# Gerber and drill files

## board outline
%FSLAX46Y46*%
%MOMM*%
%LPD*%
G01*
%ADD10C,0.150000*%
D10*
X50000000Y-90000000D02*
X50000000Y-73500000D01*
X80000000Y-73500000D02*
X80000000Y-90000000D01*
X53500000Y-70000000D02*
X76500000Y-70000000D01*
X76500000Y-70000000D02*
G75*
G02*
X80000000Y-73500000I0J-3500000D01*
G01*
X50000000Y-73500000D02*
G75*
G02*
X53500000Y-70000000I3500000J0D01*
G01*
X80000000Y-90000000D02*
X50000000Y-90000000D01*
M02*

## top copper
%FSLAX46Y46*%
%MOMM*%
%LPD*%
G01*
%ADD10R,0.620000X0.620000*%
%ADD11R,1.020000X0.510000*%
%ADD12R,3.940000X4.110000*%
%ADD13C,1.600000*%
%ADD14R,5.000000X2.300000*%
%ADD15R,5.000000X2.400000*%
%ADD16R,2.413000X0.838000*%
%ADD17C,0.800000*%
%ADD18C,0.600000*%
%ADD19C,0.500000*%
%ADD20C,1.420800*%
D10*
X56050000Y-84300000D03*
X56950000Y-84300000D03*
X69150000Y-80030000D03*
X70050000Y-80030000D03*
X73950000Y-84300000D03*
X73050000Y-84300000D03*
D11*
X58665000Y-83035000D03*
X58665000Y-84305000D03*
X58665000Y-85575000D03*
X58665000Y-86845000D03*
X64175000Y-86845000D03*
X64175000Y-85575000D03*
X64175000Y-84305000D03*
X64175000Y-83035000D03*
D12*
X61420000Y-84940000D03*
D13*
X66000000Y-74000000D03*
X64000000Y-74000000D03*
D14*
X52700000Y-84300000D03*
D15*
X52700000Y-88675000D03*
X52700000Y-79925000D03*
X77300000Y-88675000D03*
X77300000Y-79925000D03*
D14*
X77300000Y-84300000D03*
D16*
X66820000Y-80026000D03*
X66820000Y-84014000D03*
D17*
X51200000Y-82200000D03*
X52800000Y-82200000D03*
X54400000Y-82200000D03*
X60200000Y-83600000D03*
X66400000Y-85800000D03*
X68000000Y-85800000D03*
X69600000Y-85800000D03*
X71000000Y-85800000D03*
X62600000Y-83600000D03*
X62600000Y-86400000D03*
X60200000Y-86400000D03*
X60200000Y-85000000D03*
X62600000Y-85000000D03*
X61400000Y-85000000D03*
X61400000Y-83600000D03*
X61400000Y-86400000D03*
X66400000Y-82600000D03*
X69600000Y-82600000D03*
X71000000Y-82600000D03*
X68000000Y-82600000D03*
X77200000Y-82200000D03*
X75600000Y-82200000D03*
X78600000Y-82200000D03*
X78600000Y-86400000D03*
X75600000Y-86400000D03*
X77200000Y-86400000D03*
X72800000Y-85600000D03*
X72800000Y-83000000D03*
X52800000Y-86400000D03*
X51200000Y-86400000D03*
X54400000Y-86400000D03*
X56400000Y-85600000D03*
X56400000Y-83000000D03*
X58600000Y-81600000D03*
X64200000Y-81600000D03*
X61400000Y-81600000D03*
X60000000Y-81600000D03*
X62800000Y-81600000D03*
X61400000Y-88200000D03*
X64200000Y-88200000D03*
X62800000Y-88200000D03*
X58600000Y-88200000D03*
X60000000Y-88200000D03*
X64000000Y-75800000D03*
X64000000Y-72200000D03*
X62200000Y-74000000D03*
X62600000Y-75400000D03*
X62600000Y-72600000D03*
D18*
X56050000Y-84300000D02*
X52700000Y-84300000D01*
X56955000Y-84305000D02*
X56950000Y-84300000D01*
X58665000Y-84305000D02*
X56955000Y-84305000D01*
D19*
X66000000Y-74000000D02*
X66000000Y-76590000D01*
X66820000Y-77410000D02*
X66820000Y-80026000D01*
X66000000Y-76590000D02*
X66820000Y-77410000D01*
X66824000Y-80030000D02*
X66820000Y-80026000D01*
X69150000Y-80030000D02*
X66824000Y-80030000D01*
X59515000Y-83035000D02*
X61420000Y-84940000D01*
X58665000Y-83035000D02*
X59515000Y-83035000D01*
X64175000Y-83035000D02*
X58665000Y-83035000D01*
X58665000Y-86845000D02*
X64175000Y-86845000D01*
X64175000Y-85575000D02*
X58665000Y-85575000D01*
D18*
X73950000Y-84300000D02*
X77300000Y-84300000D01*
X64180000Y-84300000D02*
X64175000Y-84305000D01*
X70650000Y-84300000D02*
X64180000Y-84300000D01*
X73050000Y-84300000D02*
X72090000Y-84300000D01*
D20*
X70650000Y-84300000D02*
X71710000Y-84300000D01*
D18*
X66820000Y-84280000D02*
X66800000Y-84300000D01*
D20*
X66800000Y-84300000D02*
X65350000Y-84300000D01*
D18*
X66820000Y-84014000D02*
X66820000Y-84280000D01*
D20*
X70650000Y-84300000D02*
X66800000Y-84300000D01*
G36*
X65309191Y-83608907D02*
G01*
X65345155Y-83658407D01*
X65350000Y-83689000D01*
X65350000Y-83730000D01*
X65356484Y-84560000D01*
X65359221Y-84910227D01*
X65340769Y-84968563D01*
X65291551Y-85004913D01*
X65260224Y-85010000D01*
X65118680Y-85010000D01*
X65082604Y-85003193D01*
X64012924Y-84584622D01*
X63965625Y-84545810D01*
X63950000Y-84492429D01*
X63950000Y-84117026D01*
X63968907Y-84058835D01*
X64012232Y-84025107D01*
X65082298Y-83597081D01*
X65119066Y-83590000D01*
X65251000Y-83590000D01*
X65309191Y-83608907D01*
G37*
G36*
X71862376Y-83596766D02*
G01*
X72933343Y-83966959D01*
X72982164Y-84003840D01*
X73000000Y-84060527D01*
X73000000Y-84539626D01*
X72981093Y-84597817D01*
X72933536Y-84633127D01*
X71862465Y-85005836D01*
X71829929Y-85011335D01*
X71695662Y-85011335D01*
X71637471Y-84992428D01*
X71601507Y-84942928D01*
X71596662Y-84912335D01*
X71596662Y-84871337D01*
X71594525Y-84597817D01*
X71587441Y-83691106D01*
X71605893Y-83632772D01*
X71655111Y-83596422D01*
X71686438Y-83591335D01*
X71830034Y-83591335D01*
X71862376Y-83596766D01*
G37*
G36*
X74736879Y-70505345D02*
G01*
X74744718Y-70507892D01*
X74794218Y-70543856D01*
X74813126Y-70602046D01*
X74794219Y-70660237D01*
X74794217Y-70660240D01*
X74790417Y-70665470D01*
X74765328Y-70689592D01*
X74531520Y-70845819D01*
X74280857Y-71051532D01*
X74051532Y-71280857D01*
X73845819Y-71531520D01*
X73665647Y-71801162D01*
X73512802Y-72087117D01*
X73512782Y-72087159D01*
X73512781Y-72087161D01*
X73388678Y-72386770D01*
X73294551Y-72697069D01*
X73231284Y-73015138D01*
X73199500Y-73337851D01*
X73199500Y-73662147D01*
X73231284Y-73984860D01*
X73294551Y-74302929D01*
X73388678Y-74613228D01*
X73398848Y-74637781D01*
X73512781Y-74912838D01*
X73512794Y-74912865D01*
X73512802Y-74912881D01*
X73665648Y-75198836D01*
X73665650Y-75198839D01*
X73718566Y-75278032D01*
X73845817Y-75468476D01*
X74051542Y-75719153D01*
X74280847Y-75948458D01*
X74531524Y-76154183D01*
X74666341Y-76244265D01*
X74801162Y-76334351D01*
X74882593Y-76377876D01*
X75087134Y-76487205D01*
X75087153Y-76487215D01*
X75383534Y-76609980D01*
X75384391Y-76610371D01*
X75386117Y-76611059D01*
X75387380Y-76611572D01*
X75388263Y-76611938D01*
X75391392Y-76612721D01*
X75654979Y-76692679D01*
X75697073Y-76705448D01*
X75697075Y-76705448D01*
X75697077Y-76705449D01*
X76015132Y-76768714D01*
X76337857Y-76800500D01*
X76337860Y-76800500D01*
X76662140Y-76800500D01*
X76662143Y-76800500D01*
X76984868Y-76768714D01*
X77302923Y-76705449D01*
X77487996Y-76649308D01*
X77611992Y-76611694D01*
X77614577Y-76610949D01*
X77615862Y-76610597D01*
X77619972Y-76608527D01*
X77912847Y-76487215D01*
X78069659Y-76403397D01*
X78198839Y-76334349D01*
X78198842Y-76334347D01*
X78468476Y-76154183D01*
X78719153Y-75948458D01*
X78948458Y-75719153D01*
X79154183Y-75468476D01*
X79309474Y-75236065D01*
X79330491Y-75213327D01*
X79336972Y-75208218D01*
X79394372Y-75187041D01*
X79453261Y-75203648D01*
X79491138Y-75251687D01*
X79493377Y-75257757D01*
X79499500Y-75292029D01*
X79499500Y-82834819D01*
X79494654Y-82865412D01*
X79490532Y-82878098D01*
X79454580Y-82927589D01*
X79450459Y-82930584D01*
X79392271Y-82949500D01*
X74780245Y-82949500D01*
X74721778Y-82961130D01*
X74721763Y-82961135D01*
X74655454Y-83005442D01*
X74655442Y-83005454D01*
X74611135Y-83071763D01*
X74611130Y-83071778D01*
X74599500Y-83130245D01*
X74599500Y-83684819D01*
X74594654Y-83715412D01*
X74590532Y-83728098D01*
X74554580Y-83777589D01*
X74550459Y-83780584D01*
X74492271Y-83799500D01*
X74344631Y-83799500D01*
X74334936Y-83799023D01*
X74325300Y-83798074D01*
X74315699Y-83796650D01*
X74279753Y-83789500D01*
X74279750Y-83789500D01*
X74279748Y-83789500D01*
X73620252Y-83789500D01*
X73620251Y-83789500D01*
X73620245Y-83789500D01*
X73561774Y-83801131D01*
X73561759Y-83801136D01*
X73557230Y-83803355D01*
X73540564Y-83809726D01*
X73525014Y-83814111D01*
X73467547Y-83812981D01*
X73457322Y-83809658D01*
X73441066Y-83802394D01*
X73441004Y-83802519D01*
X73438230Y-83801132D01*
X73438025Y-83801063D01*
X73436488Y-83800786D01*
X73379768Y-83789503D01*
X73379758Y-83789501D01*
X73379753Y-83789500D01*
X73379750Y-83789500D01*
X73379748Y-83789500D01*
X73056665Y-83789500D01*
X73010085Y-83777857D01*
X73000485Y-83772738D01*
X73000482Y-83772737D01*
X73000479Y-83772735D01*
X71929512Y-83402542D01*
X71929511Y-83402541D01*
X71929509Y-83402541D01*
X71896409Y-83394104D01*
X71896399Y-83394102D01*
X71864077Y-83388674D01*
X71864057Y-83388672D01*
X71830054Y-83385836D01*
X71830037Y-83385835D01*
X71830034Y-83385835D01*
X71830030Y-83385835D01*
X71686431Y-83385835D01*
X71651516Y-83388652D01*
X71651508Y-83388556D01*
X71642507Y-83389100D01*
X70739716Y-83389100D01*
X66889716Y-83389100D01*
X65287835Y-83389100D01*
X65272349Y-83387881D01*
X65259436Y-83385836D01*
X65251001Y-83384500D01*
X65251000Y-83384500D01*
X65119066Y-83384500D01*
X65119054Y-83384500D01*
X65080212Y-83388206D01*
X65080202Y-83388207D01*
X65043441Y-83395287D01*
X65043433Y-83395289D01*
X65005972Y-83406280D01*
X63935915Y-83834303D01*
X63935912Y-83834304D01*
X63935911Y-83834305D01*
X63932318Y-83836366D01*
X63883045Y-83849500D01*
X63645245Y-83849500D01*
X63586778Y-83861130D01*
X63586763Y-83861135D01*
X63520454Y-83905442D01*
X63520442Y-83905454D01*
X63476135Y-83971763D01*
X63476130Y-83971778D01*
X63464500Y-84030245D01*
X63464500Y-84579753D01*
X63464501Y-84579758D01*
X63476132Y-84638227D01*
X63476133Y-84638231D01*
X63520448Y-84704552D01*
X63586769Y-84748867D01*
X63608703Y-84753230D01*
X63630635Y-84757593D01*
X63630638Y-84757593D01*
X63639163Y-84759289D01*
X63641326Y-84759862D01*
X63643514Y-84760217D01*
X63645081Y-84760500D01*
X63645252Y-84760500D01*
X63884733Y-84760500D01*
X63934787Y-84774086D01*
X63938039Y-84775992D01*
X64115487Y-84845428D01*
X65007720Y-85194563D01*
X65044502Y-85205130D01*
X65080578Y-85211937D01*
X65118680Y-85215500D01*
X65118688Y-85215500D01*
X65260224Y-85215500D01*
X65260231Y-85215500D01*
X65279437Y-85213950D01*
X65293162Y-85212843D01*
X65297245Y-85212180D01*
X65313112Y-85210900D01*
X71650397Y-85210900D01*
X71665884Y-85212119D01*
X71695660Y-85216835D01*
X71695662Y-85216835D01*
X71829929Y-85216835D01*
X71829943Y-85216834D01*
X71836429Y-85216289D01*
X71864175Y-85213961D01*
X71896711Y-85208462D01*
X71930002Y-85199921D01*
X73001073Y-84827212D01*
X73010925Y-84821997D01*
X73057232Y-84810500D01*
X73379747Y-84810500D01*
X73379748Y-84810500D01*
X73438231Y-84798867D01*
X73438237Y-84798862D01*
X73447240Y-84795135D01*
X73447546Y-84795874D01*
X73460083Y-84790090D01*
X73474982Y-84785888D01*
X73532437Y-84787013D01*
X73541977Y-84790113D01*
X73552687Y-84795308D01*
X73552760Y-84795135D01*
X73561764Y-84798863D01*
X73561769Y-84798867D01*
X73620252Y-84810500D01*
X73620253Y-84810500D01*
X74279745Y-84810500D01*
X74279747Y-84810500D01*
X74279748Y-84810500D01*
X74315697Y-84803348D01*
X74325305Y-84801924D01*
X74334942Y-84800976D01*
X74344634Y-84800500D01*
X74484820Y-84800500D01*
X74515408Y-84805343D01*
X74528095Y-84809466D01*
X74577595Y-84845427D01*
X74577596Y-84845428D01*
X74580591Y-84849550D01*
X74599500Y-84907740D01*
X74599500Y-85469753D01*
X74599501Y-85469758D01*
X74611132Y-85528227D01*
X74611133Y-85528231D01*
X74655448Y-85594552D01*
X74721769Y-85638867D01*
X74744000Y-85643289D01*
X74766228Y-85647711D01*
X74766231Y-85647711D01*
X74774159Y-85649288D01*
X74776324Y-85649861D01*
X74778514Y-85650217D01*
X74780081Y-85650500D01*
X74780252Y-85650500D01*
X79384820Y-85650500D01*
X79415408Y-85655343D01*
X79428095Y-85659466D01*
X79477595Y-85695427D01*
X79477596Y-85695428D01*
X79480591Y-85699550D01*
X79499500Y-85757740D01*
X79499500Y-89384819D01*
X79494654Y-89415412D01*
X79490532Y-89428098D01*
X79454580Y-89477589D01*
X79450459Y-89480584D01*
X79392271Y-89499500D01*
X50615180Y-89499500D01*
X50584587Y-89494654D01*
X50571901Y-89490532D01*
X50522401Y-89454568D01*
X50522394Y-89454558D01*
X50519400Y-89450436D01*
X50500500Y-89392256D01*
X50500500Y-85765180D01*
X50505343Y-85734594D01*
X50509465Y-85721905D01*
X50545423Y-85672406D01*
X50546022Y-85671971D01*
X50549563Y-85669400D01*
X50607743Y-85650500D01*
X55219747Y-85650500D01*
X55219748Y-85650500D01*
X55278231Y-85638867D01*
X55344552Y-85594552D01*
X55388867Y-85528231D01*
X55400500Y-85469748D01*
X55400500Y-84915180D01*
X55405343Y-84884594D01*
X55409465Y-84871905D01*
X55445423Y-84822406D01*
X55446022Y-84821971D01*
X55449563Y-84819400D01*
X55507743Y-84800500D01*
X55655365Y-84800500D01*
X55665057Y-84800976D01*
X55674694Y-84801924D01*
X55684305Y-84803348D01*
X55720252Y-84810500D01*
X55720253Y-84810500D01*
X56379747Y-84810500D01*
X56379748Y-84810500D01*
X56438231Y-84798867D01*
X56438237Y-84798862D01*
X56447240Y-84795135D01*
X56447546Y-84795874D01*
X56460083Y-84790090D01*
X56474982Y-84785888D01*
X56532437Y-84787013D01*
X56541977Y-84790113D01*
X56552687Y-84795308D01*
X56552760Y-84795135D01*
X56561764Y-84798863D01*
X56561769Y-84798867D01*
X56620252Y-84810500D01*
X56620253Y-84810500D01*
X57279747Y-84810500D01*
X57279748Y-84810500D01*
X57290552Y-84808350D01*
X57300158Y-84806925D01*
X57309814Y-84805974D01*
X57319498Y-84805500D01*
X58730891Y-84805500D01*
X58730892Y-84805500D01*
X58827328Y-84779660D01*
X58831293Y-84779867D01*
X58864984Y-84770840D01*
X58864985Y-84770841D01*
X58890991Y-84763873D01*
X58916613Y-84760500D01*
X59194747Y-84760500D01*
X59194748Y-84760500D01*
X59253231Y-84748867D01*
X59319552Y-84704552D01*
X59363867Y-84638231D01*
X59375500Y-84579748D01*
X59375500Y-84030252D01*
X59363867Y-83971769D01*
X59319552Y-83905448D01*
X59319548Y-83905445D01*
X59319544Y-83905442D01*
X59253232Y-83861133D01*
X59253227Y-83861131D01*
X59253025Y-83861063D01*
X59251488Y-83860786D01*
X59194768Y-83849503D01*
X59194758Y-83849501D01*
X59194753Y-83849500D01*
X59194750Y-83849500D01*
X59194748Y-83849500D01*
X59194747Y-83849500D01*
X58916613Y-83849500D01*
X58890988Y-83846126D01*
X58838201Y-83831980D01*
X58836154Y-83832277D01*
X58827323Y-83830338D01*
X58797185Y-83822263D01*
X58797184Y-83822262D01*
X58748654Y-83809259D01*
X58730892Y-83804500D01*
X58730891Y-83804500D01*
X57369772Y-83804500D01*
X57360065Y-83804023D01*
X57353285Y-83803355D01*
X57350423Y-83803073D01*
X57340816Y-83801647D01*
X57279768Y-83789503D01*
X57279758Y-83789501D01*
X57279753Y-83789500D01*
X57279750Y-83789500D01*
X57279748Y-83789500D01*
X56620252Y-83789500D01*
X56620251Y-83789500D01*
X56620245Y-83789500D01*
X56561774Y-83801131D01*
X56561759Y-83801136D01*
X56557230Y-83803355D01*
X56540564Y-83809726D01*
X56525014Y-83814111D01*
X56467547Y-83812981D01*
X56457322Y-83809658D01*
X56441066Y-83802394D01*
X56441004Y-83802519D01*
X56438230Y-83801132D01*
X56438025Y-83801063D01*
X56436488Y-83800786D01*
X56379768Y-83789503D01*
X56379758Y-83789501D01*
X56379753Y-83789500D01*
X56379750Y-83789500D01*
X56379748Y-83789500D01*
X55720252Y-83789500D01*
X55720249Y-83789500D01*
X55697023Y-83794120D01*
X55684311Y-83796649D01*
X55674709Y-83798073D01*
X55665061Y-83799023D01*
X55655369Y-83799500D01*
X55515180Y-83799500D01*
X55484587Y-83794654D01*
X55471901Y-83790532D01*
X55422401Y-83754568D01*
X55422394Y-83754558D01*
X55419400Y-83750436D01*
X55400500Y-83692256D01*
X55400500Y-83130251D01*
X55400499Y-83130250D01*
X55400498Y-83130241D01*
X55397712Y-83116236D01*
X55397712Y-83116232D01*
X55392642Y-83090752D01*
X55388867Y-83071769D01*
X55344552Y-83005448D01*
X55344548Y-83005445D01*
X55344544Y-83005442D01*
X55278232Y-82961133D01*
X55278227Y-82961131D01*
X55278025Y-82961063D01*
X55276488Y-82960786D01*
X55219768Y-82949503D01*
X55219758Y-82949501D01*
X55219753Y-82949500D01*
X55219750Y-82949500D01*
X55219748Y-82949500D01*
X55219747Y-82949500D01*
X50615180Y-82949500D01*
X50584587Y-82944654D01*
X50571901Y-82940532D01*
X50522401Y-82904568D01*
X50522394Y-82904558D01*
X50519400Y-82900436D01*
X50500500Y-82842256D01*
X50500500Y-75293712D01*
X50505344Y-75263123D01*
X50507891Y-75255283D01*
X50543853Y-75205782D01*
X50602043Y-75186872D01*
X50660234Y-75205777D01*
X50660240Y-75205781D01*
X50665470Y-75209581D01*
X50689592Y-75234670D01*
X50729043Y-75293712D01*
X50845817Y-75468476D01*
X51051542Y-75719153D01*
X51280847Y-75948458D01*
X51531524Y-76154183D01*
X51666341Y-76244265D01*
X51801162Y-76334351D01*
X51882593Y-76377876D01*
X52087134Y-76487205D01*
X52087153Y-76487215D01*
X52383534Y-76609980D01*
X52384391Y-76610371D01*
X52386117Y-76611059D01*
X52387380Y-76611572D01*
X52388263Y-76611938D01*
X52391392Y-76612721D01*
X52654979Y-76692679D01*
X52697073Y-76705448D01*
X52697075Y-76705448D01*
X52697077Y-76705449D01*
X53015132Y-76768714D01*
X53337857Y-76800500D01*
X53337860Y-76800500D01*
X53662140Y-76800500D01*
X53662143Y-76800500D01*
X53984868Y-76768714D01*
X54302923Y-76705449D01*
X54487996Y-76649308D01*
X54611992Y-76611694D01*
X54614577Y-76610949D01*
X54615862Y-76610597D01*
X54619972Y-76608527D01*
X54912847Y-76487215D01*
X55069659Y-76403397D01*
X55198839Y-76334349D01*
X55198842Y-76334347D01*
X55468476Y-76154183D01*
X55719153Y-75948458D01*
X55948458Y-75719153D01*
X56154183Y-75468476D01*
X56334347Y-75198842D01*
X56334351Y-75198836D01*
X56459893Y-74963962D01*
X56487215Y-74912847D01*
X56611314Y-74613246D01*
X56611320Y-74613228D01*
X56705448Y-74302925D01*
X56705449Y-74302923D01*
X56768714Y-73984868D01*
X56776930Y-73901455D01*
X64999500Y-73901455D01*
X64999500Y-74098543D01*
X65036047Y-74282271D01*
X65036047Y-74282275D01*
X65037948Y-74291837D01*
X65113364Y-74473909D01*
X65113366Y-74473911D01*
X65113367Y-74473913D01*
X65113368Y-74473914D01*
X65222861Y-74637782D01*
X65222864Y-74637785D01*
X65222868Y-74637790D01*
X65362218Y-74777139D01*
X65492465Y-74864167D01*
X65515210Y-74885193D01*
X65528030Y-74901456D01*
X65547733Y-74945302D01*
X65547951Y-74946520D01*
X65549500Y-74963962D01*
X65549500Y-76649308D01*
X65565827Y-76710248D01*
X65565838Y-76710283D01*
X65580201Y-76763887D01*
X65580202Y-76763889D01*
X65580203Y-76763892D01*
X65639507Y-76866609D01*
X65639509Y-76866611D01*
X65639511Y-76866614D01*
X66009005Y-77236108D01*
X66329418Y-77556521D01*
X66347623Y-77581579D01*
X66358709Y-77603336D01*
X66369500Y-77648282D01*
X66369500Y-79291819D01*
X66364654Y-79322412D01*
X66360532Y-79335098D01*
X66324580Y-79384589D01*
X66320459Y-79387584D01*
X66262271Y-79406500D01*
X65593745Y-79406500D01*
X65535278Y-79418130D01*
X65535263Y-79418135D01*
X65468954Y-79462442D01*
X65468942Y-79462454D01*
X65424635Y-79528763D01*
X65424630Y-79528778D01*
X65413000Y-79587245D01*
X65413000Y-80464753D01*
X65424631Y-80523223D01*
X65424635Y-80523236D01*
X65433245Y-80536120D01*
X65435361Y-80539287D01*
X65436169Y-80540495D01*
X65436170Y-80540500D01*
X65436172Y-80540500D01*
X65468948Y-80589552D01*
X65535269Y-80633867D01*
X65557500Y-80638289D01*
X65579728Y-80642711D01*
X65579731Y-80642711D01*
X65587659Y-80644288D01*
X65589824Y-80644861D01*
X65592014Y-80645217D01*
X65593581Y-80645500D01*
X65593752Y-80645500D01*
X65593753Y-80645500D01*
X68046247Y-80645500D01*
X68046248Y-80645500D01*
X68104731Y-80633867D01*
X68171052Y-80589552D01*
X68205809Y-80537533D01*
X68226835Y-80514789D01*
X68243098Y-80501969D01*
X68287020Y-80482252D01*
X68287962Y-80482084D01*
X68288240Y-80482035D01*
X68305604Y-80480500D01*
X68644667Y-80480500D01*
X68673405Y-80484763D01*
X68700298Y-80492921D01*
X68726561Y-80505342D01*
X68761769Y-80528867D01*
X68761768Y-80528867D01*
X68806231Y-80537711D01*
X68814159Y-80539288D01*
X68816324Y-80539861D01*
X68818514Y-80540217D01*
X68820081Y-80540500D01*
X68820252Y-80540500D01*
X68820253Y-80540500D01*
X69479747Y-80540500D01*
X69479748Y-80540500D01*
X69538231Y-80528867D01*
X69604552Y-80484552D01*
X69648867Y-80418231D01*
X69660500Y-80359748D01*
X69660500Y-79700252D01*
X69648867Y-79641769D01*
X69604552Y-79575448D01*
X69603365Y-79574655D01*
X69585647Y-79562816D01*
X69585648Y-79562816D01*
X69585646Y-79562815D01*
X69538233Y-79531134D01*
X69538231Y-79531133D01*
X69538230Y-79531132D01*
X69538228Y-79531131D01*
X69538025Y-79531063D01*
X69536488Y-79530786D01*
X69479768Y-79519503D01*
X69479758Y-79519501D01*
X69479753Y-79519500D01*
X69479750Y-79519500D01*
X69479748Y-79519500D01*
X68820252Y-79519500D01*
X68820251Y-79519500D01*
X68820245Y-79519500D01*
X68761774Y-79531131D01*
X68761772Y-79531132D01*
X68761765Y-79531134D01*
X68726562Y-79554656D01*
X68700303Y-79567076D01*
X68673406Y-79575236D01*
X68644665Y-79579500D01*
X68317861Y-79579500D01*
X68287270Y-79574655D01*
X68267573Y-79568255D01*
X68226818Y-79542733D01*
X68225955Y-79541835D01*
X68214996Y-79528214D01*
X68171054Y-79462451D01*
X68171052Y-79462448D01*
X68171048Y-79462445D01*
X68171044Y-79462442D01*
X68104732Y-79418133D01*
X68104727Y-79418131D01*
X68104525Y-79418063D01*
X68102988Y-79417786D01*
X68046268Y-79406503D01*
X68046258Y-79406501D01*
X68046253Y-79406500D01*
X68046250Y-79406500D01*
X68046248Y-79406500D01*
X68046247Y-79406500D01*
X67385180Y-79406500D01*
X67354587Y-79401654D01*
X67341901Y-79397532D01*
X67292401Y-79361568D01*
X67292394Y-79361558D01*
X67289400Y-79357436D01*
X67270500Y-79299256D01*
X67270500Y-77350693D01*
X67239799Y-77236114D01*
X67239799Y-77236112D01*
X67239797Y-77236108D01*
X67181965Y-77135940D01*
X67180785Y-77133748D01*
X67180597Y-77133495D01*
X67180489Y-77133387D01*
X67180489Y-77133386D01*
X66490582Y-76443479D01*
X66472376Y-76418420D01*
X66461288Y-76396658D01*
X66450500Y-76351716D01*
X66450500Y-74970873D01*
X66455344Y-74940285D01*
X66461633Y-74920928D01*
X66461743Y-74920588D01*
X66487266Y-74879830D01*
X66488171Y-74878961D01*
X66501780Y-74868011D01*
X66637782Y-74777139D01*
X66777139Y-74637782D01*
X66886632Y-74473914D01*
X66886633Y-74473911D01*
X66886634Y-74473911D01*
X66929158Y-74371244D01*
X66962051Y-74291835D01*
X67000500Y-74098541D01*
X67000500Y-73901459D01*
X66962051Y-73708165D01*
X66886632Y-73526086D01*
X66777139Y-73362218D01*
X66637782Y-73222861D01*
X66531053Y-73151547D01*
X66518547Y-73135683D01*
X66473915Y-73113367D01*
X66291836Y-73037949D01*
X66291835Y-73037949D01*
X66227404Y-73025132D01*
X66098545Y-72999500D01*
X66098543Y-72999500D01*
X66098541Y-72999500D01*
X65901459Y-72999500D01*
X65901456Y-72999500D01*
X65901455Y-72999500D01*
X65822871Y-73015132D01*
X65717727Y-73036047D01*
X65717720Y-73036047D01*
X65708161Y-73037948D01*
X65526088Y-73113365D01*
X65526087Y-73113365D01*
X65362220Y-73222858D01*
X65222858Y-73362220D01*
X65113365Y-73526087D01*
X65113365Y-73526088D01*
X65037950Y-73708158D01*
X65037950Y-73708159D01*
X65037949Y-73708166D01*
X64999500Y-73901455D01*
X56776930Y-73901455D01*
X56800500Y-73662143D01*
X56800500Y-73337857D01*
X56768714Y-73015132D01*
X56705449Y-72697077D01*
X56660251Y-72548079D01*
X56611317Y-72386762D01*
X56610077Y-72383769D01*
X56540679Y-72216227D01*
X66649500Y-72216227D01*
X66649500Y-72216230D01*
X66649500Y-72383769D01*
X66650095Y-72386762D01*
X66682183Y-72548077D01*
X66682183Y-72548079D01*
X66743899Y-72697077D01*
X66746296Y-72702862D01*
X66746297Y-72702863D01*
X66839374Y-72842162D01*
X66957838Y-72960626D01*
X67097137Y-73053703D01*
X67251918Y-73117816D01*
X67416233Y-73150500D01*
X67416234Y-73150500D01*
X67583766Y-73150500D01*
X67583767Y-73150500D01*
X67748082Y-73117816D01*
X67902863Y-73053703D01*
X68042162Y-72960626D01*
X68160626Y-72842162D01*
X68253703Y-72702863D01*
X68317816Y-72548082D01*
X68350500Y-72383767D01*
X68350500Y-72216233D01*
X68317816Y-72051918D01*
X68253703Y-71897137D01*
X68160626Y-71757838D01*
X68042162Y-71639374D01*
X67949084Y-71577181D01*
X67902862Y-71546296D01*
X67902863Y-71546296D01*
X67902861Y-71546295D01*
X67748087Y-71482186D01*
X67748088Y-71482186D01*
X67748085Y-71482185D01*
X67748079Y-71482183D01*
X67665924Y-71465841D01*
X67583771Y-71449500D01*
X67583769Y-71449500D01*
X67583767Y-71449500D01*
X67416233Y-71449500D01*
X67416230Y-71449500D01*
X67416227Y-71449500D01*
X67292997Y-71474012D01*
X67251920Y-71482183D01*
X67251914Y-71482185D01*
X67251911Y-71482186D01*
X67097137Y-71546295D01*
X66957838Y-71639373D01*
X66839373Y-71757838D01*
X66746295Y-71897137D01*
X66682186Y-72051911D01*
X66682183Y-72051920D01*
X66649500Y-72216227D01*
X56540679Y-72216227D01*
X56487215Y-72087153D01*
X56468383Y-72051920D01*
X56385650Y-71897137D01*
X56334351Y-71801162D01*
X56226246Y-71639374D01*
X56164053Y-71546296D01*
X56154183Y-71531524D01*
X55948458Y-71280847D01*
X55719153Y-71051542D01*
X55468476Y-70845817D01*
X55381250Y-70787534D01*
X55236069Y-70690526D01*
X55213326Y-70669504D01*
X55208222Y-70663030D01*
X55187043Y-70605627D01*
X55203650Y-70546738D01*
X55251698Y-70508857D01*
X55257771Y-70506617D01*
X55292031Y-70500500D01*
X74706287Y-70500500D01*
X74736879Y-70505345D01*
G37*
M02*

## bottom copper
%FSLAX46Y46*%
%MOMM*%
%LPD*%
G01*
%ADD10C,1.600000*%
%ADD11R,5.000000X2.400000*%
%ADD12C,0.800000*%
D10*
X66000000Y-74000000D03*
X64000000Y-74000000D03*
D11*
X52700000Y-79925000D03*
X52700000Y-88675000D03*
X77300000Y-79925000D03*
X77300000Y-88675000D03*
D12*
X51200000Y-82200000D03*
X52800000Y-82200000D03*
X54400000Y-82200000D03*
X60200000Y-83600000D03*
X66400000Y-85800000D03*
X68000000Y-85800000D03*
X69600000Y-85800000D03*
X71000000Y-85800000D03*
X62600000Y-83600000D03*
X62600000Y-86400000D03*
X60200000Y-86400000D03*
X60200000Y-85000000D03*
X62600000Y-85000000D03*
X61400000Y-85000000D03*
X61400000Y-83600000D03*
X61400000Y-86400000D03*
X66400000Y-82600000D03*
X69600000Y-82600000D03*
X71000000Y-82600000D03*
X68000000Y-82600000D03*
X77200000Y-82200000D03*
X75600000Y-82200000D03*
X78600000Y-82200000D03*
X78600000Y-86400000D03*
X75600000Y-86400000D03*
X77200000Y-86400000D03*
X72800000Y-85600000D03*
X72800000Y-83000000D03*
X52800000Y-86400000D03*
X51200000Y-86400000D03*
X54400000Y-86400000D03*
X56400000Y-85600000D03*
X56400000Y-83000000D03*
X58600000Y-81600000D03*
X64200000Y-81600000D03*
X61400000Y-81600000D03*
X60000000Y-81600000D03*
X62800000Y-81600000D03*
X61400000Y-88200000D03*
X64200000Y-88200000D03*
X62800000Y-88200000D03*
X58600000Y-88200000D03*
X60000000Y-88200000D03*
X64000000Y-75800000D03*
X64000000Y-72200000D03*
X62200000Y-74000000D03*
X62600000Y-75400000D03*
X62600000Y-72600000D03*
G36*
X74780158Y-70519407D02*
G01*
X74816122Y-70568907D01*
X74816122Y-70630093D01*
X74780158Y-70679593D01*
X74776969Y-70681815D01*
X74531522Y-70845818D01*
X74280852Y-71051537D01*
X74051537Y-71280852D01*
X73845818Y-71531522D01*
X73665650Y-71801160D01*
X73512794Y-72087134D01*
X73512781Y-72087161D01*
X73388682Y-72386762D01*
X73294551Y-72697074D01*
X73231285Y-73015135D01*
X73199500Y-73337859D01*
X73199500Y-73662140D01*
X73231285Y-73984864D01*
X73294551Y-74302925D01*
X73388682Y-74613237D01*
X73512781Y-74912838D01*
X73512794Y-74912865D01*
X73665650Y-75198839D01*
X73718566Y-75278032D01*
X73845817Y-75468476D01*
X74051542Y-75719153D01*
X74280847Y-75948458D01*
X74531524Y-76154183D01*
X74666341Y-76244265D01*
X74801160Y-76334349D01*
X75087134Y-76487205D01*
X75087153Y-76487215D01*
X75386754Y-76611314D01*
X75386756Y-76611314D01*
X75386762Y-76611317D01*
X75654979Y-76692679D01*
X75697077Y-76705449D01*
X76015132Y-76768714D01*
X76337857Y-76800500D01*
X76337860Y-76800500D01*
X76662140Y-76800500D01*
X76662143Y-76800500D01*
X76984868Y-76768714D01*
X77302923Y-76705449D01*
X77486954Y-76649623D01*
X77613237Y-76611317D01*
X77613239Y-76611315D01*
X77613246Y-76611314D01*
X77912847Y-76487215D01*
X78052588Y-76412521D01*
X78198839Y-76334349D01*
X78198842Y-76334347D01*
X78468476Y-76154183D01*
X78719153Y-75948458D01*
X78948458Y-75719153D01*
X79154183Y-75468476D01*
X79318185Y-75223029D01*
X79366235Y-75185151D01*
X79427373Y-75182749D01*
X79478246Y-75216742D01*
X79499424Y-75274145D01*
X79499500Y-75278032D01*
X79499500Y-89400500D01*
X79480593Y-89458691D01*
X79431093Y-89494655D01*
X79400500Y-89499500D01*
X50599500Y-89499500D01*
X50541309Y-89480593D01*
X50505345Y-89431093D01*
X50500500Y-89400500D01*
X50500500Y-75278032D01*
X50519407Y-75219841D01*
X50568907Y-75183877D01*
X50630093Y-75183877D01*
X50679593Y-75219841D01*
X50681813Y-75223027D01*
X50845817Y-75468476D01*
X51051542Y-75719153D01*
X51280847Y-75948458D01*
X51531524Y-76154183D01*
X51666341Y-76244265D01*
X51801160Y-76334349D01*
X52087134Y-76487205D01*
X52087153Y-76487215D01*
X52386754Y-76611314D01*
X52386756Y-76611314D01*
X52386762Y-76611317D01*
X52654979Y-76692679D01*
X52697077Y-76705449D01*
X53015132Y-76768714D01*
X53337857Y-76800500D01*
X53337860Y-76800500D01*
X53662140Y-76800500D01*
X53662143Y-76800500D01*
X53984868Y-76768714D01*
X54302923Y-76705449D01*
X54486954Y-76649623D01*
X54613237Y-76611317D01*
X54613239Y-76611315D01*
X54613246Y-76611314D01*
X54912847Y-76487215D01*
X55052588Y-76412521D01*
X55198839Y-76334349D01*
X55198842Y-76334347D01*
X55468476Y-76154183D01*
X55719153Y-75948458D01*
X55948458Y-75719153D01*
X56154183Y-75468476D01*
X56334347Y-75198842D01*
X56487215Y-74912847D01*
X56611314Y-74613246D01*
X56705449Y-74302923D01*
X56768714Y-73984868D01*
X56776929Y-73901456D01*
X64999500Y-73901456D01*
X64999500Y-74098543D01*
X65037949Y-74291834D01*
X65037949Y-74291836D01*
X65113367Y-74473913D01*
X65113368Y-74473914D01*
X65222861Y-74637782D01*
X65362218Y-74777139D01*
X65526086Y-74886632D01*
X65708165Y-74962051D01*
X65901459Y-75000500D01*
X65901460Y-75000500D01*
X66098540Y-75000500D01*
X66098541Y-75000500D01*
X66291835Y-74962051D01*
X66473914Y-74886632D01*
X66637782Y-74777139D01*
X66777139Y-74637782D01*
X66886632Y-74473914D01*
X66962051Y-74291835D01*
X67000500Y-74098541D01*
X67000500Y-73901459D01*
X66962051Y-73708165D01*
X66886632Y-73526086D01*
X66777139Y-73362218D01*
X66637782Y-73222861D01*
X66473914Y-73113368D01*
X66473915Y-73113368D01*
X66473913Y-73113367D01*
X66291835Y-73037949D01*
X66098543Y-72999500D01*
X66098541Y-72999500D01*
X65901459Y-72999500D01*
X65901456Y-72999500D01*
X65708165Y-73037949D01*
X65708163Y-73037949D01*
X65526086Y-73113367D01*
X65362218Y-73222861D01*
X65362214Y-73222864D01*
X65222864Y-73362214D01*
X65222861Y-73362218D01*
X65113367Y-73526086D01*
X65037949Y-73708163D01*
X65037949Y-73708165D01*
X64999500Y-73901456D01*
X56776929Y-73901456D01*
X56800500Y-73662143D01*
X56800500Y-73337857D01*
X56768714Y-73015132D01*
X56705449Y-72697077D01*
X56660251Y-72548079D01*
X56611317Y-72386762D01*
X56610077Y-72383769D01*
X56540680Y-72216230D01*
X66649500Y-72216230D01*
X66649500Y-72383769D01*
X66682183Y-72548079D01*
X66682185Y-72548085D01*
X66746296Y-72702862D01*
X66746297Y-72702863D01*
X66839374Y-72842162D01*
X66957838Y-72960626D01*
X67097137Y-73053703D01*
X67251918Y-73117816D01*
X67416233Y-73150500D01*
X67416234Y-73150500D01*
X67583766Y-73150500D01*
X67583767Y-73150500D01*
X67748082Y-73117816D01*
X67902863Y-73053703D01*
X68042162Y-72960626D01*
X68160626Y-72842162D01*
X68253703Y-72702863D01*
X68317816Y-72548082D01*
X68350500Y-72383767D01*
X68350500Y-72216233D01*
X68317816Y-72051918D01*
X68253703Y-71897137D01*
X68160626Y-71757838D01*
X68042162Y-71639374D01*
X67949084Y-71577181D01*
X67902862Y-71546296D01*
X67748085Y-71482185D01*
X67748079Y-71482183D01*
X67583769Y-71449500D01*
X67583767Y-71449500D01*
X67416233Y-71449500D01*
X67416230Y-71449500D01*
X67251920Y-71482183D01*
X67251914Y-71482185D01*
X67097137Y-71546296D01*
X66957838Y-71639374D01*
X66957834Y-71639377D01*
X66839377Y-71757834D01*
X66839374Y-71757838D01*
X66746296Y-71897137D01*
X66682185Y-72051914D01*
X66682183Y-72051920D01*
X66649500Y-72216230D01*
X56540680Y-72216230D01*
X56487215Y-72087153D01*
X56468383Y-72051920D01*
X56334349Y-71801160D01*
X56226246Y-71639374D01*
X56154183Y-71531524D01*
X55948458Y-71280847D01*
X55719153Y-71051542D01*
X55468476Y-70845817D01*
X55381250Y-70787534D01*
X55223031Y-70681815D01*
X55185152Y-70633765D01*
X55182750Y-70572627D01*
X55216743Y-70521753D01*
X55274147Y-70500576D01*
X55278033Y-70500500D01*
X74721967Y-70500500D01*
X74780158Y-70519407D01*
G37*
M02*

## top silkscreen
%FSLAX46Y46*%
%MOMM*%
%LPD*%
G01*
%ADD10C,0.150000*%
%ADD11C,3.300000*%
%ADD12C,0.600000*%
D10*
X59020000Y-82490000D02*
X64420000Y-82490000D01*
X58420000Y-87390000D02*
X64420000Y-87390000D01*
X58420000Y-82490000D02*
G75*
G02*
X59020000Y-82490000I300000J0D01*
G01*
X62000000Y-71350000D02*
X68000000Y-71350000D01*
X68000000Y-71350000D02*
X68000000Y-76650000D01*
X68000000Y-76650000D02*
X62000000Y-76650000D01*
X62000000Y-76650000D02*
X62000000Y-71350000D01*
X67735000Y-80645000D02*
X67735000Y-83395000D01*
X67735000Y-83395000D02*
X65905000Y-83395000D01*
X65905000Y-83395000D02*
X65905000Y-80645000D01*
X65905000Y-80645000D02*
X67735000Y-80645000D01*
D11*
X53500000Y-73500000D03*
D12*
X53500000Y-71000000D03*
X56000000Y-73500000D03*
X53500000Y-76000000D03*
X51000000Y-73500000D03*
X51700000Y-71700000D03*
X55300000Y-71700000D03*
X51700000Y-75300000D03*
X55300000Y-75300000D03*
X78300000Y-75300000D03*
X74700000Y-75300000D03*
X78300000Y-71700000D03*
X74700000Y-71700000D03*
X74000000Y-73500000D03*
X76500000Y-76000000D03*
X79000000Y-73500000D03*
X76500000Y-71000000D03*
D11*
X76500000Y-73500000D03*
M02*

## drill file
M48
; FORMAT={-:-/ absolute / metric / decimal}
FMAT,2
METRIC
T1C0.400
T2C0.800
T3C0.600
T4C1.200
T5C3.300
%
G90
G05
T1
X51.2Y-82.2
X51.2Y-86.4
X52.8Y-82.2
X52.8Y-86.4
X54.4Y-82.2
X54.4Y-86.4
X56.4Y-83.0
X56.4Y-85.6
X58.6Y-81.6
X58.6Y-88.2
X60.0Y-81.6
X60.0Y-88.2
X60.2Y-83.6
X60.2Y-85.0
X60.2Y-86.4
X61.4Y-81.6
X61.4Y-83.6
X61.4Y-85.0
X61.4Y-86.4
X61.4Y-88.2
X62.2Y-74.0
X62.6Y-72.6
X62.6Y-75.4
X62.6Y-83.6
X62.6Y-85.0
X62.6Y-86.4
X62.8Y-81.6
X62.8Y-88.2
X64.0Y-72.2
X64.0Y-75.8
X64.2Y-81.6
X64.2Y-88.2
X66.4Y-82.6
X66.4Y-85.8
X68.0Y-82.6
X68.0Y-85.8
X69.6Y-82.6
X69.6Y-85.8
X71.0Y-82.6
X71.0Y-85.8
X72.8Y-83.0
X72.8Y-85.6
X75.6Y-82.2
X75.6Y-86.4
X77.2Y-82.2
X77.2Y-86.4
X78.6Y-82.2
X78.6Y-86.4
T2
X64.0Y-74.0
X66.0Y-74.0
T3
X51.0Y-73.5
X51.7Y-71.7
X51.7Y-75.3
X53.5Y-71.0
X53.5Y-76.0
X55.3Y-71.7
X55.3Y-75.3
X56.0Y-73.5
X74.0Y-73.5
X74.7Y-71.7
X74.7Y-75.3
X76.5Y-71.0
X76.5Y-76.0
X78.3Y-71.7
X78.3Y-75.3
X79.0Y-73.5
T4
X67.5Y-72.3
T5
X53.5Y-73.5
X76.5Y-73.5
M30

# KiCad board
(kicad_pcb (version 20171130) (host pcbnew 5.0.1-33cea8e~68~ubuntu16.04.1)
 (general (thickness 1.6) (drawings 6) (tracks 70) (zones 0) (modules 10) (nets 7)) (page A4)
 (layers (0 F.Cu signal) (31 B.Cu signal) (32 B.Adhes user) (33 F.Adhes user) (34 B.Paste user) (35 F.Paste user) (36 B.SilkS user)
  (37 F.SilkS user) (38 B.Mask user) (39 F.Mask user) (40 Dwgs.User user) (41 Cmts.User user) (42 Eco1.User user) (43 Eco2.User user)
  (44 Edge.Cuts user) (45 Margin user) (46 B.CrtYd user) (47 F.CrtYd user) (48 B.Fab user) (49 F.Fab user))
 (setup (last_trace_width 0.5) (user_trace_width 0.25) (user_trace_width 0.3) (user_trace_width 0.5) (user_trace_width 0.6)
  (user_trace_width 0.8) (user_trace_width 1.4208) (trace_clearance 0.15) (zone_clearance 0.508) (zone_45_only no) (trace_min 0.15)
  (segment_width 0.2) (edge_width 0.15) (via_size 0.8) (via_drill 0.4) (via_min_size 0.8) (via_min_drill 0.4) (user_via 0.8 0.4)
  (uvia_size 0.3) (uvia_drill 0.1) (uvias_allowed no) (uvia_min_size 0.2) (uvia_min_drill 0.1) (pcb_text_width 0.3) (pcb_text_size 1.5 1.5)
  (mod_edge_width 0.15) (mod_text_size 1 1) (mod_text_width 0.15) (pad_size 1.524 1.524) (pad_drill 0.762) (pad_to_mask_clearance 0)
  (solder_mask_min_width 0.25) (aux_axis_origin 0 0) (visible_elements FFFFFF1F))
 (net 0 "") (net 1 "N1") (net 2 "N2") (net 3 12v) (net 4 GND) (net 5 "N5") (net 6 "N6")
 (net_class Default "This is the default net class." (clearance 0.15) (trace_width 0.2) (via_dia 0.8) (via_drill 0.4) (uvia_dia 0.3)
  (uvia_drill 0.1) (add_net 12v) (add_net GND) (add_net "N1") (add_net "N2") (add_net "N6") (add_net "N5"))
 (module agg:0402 (layer F.Cu) (at 56.5 84.3)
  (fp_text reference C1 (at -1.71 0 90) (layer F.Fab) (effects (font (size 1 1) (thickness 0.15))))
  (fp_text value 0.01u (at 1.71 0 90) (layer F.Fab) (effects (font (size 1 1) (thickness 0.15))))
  (pad 1 smd rect (at -0.45 0) (size 0.62 0.62) (layers F.Cu F.Paste F.Mask) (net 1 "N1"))
  (pad 2 smd rect (at 0.45 0) (size 0.62 0.62) (layers F.Cu F.Paste F.Mask) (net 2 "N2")))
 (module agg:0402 (layer F.Cu) (at 69.6 80.03)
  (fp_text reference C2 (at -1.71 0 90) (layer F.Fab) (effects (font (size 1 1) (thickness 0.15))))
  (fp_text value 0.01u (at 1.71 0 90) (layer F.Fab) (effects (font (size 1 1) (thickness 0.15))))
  (pad 1 smd rect (at -0.45 0) (size 0.62 0.62) (layers F.Cu F.Paste F.Mask) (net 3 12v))
  (pad 2 smd rect (at 0.45 0) (size 0.62 0.62) (layers F.Cu F.Paste F.Mask) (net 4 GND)))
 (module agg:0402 (layer F.Cu) (at 73.5 84.3)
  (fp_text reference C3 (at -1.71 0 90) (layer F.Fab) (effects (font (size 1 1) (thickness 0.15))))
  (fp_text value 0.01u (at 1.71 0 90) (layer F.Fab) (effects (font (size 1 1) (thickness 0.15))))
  (pad 2 smd rect (at 0.45 0) (size 0.62 0.62) (layers F.Cu F.Paste F.Mask) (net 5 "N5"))
  (pad 1 smd rect (at -0.45 0) (size 0.62 0.62) (layers F.Cu F.Paste F.Mask) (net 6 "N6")))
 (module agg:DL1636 (layer F.Cu) (at 61.42 84.94)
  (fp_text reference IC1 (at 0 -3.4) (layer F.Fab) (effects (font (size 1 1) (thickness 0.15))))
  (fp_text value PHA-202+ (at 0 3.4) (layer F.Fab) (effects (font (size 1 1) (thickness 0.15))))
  (fp_line (start -2.4 -2.45) (end 3 -2.45) (layer F.SilkS) (width 0.15))
  (fp_line (start -3 2.45) (end 3 2.45) (layer F.SilkS) (width 0.15))
  (fp_arc (start -2.7 -2.45) (end -3 -2.45) (angle 180) (layer F.SilkS) (width 0.15))
  (pad 1 smd rect (at -2.755 -1.905) (size 1.02 0.51) (layers F.Cu F.Paste F.Mask) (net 4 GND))
  (pad 2 smd rect (at -2.755 -0.635) (size 1.02 0.51) (layers F.Cu F.Paste F.Mask) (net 2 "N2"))
  (pad 3 smd rect (at -2.755 0.635) (size 1.02 0.51) (layers F.Cu F.Paste F.Mask) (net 4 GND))
  (pad 4 smd rect (at -2.755 1.905) (size 1.02 0.51) (layers F.Cu F.Paste F.Mask) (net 4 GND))
  (pad 5 smd rect (at 2.755 1.905) (size 1.02 0.51) (layers F.Cu F.Paste F.Mask) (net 4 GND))
  (pad 6 smd rect (at 2.755 0.635) (size 1.02 0.51) (layers F.Cu F.Paste F.Mask) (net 4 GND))
  (pad 7 smd rect (at 2.755 -0.635) (size 1.02 0.51) (layers F.Cu F.Paste F.Mask) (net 6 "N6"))
  (pad 8 smd rect (at 2.755 -1.905) (size 1.02 0.51) (layers F.Cu F.Paste F.Mask) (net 4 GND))
  (pad EP smd rect (at 0 0) (size 3.94 4.11) (layers F.Cu F.Paste F.Mask) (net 4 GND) (solder_mask_margin 0.001) (solder_paste_margin 0.001)))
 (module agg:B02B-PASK (layer F.Cu) (at 65 74)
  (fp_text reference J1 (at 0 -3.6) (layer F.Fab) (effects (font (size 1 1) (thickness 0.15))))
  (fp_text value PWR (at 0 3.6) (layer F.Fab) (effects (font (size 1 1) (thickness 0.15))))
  (fp_line (start -3 -2.65) (end 3 -2.65) (layer F.SilkS) (width 0.15))
  (fp_line (start 3 -2.65) (end 3 2.65) (layer F.SilkS) (width 0.15))
  (fp_line (start 3 2.65) (end -3 2.65) (layer F.SilkS) (width 0.15))
  (fp_line (start -3 2.65) (end -3 -2.65) (layer F.SilkS) (width 0.15))
  (pad "" np_thru_hole circle (at 2.5 -1.7) (size 1.2 1.2) (drill 1.2) (layers *.Mask))
  (pad 1 thru_hole circle (at 1 0) (size 1.6 1.6) (drill 0.8) (layers *.Cu *.Mask) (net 3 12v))
  (pad 2 thru_hole circle (at -1 0) (size 1.6 1.6) (drill 0.8) (layers *.Cu *.Mask) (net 4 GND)))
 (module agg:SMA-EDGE (layer F.Cu) (at 52.7 84.3 90)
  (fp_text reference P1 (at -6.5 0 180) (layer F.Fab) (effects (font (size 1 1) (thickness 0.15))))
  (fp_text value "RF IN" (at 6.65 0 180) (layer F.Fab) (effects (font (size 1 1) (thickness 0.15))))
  (pad 1 smd rect (at 0 0 90) (size 2.3 5) (layers F.Cu F.Paste F.Mask) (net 1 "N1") (zone_connect 2))
  (pad 2 smd rect (at 4.375 0 90) (size 2.4 5) (layers B.Cu B.Paste B.Mask) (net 4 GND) (zone_connect 2))
  (pad 2 smd rect (at -4.375 0 90) (size 2.4 5) (layers B.Cu B.Paste B.Mask) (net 4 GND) (zone_connect 2))
  (pad 2 smd rect (at -4.375 0 90) (size 2.4 5) (layers F.Cu F.Paste F.Mask) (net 4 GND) (zone_connect 2))
  (pad 2 smd rect (at 4.375 0 90) (size 2.4 5) (layers F.Cu F.Paste F.Mask) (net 4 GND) (zone_connect 2)))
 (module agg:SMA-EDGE (layer F.Cu) (at 77.3 84.3 270)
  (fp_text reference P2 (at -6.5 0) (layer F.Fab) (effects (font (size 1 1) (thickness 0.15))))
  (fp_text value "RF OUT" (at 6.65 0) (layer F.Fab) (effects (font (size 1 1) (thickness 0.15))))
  (pad 2 smd rect (at 4.375 0 270) (size 2.4 5) (layers F.Cu F.Paste F.Mask) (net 4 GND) (zone_connect 2))
  (pad 2 smd rect (at -4.375 0 270) (size 2.4 5) (layers F.Cu F.Paste F.Mask) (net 4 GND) (zone_connect 2))
  (pad 2 smd rect (at -4.375 0 270) (size 2.4 5) (layers B.Cu B.Paste B.Mask) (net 4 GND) (zone_connect 2))
  (pad 2 smd rect (at 4.375 0 270) (size 2.4 5) (layers B.Cu B.Paste B.Mask) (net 4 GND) (zone_connect 2))
  (pad 1 smd rect (at 0 0 270) (size 2.3 5) (layers F.Cu F.Paste F.Mask) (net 5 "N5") (zone_connect 2)))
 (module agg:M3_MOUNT (layer F.Cu) (at 53.5 73.5)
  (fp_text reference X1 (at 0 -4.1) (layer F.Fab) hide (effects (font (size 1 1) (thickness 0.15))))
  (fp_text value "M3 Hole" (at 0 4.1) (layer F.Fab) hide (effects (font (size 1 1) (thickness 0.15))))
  (pad "" np_thru_hole circle (at 0 0) (size 3.3 3.3) (drill 3.3) (layers *.Cu *.Mask F.SilkS) (solder_mask_margin 1.5) (clearance 1.65))
  (pad "" np_thru_hole circle (at 0 -2.5) (size 0.6 0.6) (drill 0.6) (layers *.Cu *.Mask F.SilkS))
  (pad "" np_thru_hole circle (at 2.5 0) (size 0.6 0.6) (drill 0.6) (layers *.Cu *.Mask F.SilkS))
  (pad "" np_thru_hole circle (at 0 2.5) (size 0.6 0.6) (drill 0.6) (layers *.Cu *.Mask F.SilkS))
  (pad "" np_thru_hole circle (at -2.5 0) (size 0.6 0.6) (drill 0.6) (layers *.Cu *.Mask F.SilkS))
  (pad "" np_thru_hole circle (at -1.8 -1.8) (size 0.6 0.6) (drill 0.6) (layers *.Cu *.Mask F.SilkS))
  (pad "" np_thru_hole circle (at 1.8 -1.8) (size 0.6 0.6) (drill 0.6) (layers *.Cu *.Mask F.SilkS))
  (pad "" np_thru_hole circle (at -1.8 1.8) (size 0.6 0.6) (drill 0.6) (layers *.Cu *.Mask F.SilkS))
  (pad "" np_thru_hole circle (at 1.8 1.8) (size 0.6 0.6) (drill 0.6) (layers *.Cu *.Mask F.SilkS)))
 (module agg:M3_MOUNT (layer F.Cu) (at 76.5 73.5)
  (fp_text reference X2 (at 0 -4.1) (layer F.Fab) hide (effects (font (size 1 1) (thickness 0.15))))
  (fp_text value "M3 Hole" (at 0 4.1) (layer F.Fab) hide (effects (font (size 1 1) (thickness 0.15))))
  (pad "" np_thru_hole circle (at 1.8 1.8) (size 0.6 0.6) (drill 0.6) (layers *.Cu *.Mask F.SilkS))
  (pad "" np_thru_hole circle (at -1.8 1.8) (size 0.6 0.6) (drill 0.6) (layers *.Cu *.Mask F.SilkS))
  (pad "" np_thru_hole circle (at 1.8 -1.8) (size 0.6 0.6) (drill 0.6) (layers *.Cu *.Mask F.SilkS))
  (pad "" np_thru_hole circle (at -1.8 -1.8) (size 0.6 0.6) (drill 0.6) (layers *.Cu *.Mask F.SilkS))
  (pad "" np_thru_hole circle (at -2.5 0) (size 0.6 0.6) (drill 0.6) (layers *.Cu *.Mask F.SilkS))
  (pad "" np_thru_hole circle (at 0 2.5) (size 0.6 0.6) (drill 0.6) (layers *.Cu *.Mask F.SilkS))
  (pad "" np_thru_hole circle (at 2.5 0) (size 0.6 0.6) (drill 0.6) (layers *.Cu *.Mask F.SilkS))
  (pad "" np_thru_hole circle (at 0 -2.5) (size 0.6 0.6) (drill 0.6) (layers *.Cu *.Mask F.SilkS))
  (pad "" np_thru_hole circle (at 0 0) (size 3.3 3.3) (drill 3.3) (layers *.Cu *.Mask F.SilkS) (solder_mask_margin 1.5) (clearance 1.65)))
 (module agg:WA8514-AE (layer F.Cu) (at 66.82 82.02 270)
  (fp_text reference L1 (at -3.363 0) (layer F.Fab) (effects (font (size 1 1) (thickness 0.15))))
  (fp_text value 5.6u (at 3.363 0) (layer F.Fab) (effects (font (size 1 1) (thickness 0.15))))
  (fp_line (start -1.375 -0.915) (end 1.375 -0.915) (layer F.SilkS) (width 0.15))
  (fp_line (start 1.375 -0.915) (end 1.375 0.915) (layer F.SilkS) (width 0.15))
  (fp_line (start 1.375 0.915) (end -1.375 0.915) (layer F.SilkS) (width 0.15))
  (fp_line (start -1.375 0.915) (end -1.375 -0.915) (layer F.SilkS) (width 0.15))
  (pad 1 smd rect (at -1.994 0 270) (size 0.838 2.413) (layers F.Cu F.Paste F.Mask) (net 3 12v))
  (pad 2 smd rect (at 1.994 0 270) (size 0.838 2.413) (layers F.Cu F.Paste F.Mask) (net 6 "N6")))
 (gr_line (start 50 90) (end 50 73.5) (layer Edge.Cuts) (width 0.15))
 (gr_line (start 80 73.5) (end 80 90) (layer Edge.Cuts) (width 0.15))
 (gr_line (start 53.5 70) (end 76.5 70) (layer Edge.Cuts) (width 0.15))
 (gr_arc (start 76.5 73.5) (end 80 73.5) (angle -90) (layer Edge.Cuts) (width 0.15))
 (gr_arc (start 53.5 73.5) (end 53.5 70) (angle -90) (layer Edge.Cuts) (width 0.15))
 (gr_line (start 80 90) (end 50 90) (layer Edge.Cuts) (width 0.15))
 (segment (start 56.05 84.3) (end 52.7 84.3) (width 0.6) (layer F.Cu) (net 1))
 (segment (start 56.955 84.305) (end 56.95 84.3) (width 0.6) (layer F.Cu) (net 2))
 (segment (start 58.665 84.305) (end 56.955 84.305) (width 0.6) (layer F.Cu) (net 2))
 (segment (start 66 74) (end 66 76.59) (width 0.5) (layer F.Cu) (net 3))
 (segment (start 66.82 77.41) (end 66.82 80.026) (width 0.5) (layer F.Cu) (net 3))
 (segment (start 66 76.59) (end 66.82 77.41) (width 0.5) (layer F.Cu) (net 3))
 (segment (start 66.824 80.03) (end 66.82 80.026) (width 0.5) (layer F.Cu) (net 3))
 (segment (start 69.15 80.03) (end 66.824 80.03) (width 0.5) (layer F.Cu) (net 3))
 (segment (start 59.515 83.035) (end 61.42 84.94) (width 0.5) (layer F.Cu) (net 4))
 (segment (start 58.665 83.035) (end 59.515 83.035) (width 0.5) (layer F.Cu) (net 4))
 (segment (start 64.175 83.035) (end 58.665 83.035) (width 0.5) (layer F.Cu) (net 4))
 (segment (start 58.665 86.845) (end 64.175 86.845) (width 0.5) (layer F.Cu) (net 4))
 (segment (start 64.175 85.575) (end 58.665 85.575) (width 0.5) (layer F.Cu) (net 4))
 (via (at 51.2 82.2) (size 0.8) (drill 0.4) (layers F.Cu B.Cu) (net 4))
 (via (at 52.8 82.2) (size 0.8) (drill 0.4) (layers F.Cu B.Cu) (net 4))
 (via (at 54.4 82.2) (size 0.8) (drill 0.4) (layers F.Cu B.Cu) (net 4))
 (via (at 60.2 83.6) (size 0.8) (drill 0.4) (layers F.Cu B.Cu) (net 4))
 (via (at 66.4 85.8) (size 0.8) (drill 0.4) (layers F.Cu B.Cu) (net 4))
 (via (at 68 85.8) (size 0.8) (drill 0.4) (layers F.Cu B.Cu) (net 4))
 (via (at 69.6 85.8) (size 0.8) (drill 0.4) (layers F.Cu B.Cu) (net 4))
 (via (at 71 85.8) (size 0.8) (drill 0.4) (layers F.Cu B.Cu) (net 4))
 (via (at 62.6 83.6) (size 0.8) (drill 0.4) (layers F.Cu B.Cu) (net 4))
 (via (at 62.6 86.4) (size 0.8) (drill 0.4) (layers F.Cu B.Cu) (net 4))
 (via (at 60.2 86.4) (size 0.8) (drill 0.4) (layers F.Cu B.Cu) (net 4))
 (via (at 60.2 85) (size 0.8) (drill 0.4) (layers F.Cu B.Cu) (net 4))
 (via (at 62.6 85) (size 0.8) (drill 0.4) (layers F.Cu B.Cu) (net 4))
 (via (at 61.4 85) (size 0.8) (drill 0.4) (layers F.Cu B.Cu) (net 4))
 (via (at 61.4 83.6) (size 0.8) (drill 0.4) (layers F.Cu B.Cu) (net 4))
 (via (at 61.4 86.4) (size 0.8) (drill 0.4) (layers F.Cu B.Cu) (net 4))
 (via (at 66.4 82.6) (size 0.8) (drill 0.4) (layers F.Cu B.Cu) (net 4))
 (via (at 69.6 82.6) (size 0.8) (drill 0.4) (layers F.Cu B.Cu) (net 4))
 (via (at 71 82.6) (size 0.8) (drill 0.4) (layers F.Cu B.Cu) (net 4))
 (via (at 68 82.6) (size 0.8) (drill 0.4) (layers F.Cu B.Cu) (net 4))
 (via (at 77.2 82.2) (size 0.8) (drill 0.4) (layers F.Cu B.Cu) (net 4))
 (via (at 75.6 82.2) (size 0.8) (drill 0.4) (layers F.Cu B.Cu) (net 4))
 (via (at 78.6 82.2) (size 0.8) (drill 0.4) (layers F.Cu B.Cu) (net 4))
 (via (at 78.6 86.4) (size 0.8) (drill 0.4) (layers F.Cu B.Cu) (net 4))
 (via (at 75.6 86.4) (size 0.8) (drill 0.4) (layers F.Cu B.Cu) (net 4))
 (via (at 77.2 86.4) (size 0.8) (drill 0.4) (layers F.Cu B.Cu) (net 4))
 (via (at 72.8 85.6) (size 0.8) (drill 0.4) (layers F.Cu B.Cu) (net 4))
 (via (at 72.8 83) (size 0.8) (drill 0.4) (layers F.Cu B.Cu) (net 4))
 (via (at 52.8 86.4) (size 0.8) (drill 0.4) (layers F.Cu B.Cu) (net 4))
 (via (at 51.2 86.4) (size 0.8) (drill 0.4) (layers F.Cu B.Cu) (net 4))
 (via (at 54.4 86.4) (size 0.8) (drill 0.4) (layers F.Cu B.Cu) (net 4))
 (via (at 56.4 85.6) (size 0.8) (drill 0.4) (layers F.Cu B.Cu) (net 4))
 (via (at 56.4 83) (size 0.8) (drill 0.4) (layers F.Cu B.Cu) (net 4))
 (via (at 58.6 81.6) (size 0.8) (drill 0.4) (layers F.Cu B.Cu) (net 4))
 (via (at 64.2 81.6) (size 0.8) (drill 0.4) (layers F.Cu B.Cu) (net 4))
 (via (at 61.4 81.6) (size 0.8) (drill 0.4) (layers F.Cu B.Cu) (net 4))
 (via (at 60 81.6) (size 0.8) (drill 0.4) (layers F.Cu B.Cu) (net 4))
 (via (at 62.8 81.6) (size 0.8) (drill 0.4) (layers F.Cu B.Cu) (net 4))
 (via (at 61.4 88.2) (size 0.8) (drill 0.4) (layers F.Cu B.Cu) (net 4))
 (via (at 64.2 88.2) (size 0.8) (drill 0.4) (layers F.Cu B.Cu) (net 4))
 (via (at 62.8 88.2) (size 0.8) (drill 0.4) (layers F.Cu B.Cu) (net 4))
 (via (at 58.6 88.2) (size 0.8) (drill 0.4) (layers F.Cu B.Cu) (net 4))
 (via (at 60 88.2) (size 0.8) (drill 0.4) (layers F.Cu B.Cu) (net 4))
 (via (at 64 75.8) (size 0.8) (drill 0.4) (layers F.Cu B.Cu) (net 4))
 (via (at 64 72.2) (size 0.8) (drill 0.4) (layers F.Cu B.Cu) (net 4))
 (via (at 62.2 74) (size 0.8) (drill 0.4) (layers F.Cu B.Cu) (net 4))
 (via (at 62.6 75.4) (size 0.8) (drill 0.4) (layers F.Cu B.Cu) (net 4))
 (via (at 62.6 72.6) (size 0.8) (drill 0.4) (layers F.Cu B.Cu) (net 4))
 (segment (start 73.95 84.3) (end 77.3 84.3) (width 0.6) (layer F.Cu) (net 5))
 (segment (start 64.18 84.3) (end 64.175 84.305) (width 0.6) (layer F.Cu) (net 6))
 (segment (start 70.65 84.3) (end 64.18 84.3) (width 0.6) (layer F.Cu) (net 6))
 (segment (start 73.05 84.3) (end 72.09 84.3) (width 0.6) (layer F.Cu) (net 6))
 (segment (start 70.65 84.3) (end 71.71 84.3) (width 1.4208) (layer F.Cu) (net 6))
 (segment (start 66.82 84.28) (end 66.8 84.3) (width 0.6) (layer F.Cu) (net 6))
 (segment (start 66.8 84.3) (end 65.35 84.3) (width 1.4208) (layer F.Cu) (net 6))
 (segment (start 66.82 84.014) (end 66.82 84.28) (width 0.6) (layer F.Cu) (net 6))
 (segment (start 70.65 84.3) (end 66.8 84.3) (width 1.4208) (layer F.Cu) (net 6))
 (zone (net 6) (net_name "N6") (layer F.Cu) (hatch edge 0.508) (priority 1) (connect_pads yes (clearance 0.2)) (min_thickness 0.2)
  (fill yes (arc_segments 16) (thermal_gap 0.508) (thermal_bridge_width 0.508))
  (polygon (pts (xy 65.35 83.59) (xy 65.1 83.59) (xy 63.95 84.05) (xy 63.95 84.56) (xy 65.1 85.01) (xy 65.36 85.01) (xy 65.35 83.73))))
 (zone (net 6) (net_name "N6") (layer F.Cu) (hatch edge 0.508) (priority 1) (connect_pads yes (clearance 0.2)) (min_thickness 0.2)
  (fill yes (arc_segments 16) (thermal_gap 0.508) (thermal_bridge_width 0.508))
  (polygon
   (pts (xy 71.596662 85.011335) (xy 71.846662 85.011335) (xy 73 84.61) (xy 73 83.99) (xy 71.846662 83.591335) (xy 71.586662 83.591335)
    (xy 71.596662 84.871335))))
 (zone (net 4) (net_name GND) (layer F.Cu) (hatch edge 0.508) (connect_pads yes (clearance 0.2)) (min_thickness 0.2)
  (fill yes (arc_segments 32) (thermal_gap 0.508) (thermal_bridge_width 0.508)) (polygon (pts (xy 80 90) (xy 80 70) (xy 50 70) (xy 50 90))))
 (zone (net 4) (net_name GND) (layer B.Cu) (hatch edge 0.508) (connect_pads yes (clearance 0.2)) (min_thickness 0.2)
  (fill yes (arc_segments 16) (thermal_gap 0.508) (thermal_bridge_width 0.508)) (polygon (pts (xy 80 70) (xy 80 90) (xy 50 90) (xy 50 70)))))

